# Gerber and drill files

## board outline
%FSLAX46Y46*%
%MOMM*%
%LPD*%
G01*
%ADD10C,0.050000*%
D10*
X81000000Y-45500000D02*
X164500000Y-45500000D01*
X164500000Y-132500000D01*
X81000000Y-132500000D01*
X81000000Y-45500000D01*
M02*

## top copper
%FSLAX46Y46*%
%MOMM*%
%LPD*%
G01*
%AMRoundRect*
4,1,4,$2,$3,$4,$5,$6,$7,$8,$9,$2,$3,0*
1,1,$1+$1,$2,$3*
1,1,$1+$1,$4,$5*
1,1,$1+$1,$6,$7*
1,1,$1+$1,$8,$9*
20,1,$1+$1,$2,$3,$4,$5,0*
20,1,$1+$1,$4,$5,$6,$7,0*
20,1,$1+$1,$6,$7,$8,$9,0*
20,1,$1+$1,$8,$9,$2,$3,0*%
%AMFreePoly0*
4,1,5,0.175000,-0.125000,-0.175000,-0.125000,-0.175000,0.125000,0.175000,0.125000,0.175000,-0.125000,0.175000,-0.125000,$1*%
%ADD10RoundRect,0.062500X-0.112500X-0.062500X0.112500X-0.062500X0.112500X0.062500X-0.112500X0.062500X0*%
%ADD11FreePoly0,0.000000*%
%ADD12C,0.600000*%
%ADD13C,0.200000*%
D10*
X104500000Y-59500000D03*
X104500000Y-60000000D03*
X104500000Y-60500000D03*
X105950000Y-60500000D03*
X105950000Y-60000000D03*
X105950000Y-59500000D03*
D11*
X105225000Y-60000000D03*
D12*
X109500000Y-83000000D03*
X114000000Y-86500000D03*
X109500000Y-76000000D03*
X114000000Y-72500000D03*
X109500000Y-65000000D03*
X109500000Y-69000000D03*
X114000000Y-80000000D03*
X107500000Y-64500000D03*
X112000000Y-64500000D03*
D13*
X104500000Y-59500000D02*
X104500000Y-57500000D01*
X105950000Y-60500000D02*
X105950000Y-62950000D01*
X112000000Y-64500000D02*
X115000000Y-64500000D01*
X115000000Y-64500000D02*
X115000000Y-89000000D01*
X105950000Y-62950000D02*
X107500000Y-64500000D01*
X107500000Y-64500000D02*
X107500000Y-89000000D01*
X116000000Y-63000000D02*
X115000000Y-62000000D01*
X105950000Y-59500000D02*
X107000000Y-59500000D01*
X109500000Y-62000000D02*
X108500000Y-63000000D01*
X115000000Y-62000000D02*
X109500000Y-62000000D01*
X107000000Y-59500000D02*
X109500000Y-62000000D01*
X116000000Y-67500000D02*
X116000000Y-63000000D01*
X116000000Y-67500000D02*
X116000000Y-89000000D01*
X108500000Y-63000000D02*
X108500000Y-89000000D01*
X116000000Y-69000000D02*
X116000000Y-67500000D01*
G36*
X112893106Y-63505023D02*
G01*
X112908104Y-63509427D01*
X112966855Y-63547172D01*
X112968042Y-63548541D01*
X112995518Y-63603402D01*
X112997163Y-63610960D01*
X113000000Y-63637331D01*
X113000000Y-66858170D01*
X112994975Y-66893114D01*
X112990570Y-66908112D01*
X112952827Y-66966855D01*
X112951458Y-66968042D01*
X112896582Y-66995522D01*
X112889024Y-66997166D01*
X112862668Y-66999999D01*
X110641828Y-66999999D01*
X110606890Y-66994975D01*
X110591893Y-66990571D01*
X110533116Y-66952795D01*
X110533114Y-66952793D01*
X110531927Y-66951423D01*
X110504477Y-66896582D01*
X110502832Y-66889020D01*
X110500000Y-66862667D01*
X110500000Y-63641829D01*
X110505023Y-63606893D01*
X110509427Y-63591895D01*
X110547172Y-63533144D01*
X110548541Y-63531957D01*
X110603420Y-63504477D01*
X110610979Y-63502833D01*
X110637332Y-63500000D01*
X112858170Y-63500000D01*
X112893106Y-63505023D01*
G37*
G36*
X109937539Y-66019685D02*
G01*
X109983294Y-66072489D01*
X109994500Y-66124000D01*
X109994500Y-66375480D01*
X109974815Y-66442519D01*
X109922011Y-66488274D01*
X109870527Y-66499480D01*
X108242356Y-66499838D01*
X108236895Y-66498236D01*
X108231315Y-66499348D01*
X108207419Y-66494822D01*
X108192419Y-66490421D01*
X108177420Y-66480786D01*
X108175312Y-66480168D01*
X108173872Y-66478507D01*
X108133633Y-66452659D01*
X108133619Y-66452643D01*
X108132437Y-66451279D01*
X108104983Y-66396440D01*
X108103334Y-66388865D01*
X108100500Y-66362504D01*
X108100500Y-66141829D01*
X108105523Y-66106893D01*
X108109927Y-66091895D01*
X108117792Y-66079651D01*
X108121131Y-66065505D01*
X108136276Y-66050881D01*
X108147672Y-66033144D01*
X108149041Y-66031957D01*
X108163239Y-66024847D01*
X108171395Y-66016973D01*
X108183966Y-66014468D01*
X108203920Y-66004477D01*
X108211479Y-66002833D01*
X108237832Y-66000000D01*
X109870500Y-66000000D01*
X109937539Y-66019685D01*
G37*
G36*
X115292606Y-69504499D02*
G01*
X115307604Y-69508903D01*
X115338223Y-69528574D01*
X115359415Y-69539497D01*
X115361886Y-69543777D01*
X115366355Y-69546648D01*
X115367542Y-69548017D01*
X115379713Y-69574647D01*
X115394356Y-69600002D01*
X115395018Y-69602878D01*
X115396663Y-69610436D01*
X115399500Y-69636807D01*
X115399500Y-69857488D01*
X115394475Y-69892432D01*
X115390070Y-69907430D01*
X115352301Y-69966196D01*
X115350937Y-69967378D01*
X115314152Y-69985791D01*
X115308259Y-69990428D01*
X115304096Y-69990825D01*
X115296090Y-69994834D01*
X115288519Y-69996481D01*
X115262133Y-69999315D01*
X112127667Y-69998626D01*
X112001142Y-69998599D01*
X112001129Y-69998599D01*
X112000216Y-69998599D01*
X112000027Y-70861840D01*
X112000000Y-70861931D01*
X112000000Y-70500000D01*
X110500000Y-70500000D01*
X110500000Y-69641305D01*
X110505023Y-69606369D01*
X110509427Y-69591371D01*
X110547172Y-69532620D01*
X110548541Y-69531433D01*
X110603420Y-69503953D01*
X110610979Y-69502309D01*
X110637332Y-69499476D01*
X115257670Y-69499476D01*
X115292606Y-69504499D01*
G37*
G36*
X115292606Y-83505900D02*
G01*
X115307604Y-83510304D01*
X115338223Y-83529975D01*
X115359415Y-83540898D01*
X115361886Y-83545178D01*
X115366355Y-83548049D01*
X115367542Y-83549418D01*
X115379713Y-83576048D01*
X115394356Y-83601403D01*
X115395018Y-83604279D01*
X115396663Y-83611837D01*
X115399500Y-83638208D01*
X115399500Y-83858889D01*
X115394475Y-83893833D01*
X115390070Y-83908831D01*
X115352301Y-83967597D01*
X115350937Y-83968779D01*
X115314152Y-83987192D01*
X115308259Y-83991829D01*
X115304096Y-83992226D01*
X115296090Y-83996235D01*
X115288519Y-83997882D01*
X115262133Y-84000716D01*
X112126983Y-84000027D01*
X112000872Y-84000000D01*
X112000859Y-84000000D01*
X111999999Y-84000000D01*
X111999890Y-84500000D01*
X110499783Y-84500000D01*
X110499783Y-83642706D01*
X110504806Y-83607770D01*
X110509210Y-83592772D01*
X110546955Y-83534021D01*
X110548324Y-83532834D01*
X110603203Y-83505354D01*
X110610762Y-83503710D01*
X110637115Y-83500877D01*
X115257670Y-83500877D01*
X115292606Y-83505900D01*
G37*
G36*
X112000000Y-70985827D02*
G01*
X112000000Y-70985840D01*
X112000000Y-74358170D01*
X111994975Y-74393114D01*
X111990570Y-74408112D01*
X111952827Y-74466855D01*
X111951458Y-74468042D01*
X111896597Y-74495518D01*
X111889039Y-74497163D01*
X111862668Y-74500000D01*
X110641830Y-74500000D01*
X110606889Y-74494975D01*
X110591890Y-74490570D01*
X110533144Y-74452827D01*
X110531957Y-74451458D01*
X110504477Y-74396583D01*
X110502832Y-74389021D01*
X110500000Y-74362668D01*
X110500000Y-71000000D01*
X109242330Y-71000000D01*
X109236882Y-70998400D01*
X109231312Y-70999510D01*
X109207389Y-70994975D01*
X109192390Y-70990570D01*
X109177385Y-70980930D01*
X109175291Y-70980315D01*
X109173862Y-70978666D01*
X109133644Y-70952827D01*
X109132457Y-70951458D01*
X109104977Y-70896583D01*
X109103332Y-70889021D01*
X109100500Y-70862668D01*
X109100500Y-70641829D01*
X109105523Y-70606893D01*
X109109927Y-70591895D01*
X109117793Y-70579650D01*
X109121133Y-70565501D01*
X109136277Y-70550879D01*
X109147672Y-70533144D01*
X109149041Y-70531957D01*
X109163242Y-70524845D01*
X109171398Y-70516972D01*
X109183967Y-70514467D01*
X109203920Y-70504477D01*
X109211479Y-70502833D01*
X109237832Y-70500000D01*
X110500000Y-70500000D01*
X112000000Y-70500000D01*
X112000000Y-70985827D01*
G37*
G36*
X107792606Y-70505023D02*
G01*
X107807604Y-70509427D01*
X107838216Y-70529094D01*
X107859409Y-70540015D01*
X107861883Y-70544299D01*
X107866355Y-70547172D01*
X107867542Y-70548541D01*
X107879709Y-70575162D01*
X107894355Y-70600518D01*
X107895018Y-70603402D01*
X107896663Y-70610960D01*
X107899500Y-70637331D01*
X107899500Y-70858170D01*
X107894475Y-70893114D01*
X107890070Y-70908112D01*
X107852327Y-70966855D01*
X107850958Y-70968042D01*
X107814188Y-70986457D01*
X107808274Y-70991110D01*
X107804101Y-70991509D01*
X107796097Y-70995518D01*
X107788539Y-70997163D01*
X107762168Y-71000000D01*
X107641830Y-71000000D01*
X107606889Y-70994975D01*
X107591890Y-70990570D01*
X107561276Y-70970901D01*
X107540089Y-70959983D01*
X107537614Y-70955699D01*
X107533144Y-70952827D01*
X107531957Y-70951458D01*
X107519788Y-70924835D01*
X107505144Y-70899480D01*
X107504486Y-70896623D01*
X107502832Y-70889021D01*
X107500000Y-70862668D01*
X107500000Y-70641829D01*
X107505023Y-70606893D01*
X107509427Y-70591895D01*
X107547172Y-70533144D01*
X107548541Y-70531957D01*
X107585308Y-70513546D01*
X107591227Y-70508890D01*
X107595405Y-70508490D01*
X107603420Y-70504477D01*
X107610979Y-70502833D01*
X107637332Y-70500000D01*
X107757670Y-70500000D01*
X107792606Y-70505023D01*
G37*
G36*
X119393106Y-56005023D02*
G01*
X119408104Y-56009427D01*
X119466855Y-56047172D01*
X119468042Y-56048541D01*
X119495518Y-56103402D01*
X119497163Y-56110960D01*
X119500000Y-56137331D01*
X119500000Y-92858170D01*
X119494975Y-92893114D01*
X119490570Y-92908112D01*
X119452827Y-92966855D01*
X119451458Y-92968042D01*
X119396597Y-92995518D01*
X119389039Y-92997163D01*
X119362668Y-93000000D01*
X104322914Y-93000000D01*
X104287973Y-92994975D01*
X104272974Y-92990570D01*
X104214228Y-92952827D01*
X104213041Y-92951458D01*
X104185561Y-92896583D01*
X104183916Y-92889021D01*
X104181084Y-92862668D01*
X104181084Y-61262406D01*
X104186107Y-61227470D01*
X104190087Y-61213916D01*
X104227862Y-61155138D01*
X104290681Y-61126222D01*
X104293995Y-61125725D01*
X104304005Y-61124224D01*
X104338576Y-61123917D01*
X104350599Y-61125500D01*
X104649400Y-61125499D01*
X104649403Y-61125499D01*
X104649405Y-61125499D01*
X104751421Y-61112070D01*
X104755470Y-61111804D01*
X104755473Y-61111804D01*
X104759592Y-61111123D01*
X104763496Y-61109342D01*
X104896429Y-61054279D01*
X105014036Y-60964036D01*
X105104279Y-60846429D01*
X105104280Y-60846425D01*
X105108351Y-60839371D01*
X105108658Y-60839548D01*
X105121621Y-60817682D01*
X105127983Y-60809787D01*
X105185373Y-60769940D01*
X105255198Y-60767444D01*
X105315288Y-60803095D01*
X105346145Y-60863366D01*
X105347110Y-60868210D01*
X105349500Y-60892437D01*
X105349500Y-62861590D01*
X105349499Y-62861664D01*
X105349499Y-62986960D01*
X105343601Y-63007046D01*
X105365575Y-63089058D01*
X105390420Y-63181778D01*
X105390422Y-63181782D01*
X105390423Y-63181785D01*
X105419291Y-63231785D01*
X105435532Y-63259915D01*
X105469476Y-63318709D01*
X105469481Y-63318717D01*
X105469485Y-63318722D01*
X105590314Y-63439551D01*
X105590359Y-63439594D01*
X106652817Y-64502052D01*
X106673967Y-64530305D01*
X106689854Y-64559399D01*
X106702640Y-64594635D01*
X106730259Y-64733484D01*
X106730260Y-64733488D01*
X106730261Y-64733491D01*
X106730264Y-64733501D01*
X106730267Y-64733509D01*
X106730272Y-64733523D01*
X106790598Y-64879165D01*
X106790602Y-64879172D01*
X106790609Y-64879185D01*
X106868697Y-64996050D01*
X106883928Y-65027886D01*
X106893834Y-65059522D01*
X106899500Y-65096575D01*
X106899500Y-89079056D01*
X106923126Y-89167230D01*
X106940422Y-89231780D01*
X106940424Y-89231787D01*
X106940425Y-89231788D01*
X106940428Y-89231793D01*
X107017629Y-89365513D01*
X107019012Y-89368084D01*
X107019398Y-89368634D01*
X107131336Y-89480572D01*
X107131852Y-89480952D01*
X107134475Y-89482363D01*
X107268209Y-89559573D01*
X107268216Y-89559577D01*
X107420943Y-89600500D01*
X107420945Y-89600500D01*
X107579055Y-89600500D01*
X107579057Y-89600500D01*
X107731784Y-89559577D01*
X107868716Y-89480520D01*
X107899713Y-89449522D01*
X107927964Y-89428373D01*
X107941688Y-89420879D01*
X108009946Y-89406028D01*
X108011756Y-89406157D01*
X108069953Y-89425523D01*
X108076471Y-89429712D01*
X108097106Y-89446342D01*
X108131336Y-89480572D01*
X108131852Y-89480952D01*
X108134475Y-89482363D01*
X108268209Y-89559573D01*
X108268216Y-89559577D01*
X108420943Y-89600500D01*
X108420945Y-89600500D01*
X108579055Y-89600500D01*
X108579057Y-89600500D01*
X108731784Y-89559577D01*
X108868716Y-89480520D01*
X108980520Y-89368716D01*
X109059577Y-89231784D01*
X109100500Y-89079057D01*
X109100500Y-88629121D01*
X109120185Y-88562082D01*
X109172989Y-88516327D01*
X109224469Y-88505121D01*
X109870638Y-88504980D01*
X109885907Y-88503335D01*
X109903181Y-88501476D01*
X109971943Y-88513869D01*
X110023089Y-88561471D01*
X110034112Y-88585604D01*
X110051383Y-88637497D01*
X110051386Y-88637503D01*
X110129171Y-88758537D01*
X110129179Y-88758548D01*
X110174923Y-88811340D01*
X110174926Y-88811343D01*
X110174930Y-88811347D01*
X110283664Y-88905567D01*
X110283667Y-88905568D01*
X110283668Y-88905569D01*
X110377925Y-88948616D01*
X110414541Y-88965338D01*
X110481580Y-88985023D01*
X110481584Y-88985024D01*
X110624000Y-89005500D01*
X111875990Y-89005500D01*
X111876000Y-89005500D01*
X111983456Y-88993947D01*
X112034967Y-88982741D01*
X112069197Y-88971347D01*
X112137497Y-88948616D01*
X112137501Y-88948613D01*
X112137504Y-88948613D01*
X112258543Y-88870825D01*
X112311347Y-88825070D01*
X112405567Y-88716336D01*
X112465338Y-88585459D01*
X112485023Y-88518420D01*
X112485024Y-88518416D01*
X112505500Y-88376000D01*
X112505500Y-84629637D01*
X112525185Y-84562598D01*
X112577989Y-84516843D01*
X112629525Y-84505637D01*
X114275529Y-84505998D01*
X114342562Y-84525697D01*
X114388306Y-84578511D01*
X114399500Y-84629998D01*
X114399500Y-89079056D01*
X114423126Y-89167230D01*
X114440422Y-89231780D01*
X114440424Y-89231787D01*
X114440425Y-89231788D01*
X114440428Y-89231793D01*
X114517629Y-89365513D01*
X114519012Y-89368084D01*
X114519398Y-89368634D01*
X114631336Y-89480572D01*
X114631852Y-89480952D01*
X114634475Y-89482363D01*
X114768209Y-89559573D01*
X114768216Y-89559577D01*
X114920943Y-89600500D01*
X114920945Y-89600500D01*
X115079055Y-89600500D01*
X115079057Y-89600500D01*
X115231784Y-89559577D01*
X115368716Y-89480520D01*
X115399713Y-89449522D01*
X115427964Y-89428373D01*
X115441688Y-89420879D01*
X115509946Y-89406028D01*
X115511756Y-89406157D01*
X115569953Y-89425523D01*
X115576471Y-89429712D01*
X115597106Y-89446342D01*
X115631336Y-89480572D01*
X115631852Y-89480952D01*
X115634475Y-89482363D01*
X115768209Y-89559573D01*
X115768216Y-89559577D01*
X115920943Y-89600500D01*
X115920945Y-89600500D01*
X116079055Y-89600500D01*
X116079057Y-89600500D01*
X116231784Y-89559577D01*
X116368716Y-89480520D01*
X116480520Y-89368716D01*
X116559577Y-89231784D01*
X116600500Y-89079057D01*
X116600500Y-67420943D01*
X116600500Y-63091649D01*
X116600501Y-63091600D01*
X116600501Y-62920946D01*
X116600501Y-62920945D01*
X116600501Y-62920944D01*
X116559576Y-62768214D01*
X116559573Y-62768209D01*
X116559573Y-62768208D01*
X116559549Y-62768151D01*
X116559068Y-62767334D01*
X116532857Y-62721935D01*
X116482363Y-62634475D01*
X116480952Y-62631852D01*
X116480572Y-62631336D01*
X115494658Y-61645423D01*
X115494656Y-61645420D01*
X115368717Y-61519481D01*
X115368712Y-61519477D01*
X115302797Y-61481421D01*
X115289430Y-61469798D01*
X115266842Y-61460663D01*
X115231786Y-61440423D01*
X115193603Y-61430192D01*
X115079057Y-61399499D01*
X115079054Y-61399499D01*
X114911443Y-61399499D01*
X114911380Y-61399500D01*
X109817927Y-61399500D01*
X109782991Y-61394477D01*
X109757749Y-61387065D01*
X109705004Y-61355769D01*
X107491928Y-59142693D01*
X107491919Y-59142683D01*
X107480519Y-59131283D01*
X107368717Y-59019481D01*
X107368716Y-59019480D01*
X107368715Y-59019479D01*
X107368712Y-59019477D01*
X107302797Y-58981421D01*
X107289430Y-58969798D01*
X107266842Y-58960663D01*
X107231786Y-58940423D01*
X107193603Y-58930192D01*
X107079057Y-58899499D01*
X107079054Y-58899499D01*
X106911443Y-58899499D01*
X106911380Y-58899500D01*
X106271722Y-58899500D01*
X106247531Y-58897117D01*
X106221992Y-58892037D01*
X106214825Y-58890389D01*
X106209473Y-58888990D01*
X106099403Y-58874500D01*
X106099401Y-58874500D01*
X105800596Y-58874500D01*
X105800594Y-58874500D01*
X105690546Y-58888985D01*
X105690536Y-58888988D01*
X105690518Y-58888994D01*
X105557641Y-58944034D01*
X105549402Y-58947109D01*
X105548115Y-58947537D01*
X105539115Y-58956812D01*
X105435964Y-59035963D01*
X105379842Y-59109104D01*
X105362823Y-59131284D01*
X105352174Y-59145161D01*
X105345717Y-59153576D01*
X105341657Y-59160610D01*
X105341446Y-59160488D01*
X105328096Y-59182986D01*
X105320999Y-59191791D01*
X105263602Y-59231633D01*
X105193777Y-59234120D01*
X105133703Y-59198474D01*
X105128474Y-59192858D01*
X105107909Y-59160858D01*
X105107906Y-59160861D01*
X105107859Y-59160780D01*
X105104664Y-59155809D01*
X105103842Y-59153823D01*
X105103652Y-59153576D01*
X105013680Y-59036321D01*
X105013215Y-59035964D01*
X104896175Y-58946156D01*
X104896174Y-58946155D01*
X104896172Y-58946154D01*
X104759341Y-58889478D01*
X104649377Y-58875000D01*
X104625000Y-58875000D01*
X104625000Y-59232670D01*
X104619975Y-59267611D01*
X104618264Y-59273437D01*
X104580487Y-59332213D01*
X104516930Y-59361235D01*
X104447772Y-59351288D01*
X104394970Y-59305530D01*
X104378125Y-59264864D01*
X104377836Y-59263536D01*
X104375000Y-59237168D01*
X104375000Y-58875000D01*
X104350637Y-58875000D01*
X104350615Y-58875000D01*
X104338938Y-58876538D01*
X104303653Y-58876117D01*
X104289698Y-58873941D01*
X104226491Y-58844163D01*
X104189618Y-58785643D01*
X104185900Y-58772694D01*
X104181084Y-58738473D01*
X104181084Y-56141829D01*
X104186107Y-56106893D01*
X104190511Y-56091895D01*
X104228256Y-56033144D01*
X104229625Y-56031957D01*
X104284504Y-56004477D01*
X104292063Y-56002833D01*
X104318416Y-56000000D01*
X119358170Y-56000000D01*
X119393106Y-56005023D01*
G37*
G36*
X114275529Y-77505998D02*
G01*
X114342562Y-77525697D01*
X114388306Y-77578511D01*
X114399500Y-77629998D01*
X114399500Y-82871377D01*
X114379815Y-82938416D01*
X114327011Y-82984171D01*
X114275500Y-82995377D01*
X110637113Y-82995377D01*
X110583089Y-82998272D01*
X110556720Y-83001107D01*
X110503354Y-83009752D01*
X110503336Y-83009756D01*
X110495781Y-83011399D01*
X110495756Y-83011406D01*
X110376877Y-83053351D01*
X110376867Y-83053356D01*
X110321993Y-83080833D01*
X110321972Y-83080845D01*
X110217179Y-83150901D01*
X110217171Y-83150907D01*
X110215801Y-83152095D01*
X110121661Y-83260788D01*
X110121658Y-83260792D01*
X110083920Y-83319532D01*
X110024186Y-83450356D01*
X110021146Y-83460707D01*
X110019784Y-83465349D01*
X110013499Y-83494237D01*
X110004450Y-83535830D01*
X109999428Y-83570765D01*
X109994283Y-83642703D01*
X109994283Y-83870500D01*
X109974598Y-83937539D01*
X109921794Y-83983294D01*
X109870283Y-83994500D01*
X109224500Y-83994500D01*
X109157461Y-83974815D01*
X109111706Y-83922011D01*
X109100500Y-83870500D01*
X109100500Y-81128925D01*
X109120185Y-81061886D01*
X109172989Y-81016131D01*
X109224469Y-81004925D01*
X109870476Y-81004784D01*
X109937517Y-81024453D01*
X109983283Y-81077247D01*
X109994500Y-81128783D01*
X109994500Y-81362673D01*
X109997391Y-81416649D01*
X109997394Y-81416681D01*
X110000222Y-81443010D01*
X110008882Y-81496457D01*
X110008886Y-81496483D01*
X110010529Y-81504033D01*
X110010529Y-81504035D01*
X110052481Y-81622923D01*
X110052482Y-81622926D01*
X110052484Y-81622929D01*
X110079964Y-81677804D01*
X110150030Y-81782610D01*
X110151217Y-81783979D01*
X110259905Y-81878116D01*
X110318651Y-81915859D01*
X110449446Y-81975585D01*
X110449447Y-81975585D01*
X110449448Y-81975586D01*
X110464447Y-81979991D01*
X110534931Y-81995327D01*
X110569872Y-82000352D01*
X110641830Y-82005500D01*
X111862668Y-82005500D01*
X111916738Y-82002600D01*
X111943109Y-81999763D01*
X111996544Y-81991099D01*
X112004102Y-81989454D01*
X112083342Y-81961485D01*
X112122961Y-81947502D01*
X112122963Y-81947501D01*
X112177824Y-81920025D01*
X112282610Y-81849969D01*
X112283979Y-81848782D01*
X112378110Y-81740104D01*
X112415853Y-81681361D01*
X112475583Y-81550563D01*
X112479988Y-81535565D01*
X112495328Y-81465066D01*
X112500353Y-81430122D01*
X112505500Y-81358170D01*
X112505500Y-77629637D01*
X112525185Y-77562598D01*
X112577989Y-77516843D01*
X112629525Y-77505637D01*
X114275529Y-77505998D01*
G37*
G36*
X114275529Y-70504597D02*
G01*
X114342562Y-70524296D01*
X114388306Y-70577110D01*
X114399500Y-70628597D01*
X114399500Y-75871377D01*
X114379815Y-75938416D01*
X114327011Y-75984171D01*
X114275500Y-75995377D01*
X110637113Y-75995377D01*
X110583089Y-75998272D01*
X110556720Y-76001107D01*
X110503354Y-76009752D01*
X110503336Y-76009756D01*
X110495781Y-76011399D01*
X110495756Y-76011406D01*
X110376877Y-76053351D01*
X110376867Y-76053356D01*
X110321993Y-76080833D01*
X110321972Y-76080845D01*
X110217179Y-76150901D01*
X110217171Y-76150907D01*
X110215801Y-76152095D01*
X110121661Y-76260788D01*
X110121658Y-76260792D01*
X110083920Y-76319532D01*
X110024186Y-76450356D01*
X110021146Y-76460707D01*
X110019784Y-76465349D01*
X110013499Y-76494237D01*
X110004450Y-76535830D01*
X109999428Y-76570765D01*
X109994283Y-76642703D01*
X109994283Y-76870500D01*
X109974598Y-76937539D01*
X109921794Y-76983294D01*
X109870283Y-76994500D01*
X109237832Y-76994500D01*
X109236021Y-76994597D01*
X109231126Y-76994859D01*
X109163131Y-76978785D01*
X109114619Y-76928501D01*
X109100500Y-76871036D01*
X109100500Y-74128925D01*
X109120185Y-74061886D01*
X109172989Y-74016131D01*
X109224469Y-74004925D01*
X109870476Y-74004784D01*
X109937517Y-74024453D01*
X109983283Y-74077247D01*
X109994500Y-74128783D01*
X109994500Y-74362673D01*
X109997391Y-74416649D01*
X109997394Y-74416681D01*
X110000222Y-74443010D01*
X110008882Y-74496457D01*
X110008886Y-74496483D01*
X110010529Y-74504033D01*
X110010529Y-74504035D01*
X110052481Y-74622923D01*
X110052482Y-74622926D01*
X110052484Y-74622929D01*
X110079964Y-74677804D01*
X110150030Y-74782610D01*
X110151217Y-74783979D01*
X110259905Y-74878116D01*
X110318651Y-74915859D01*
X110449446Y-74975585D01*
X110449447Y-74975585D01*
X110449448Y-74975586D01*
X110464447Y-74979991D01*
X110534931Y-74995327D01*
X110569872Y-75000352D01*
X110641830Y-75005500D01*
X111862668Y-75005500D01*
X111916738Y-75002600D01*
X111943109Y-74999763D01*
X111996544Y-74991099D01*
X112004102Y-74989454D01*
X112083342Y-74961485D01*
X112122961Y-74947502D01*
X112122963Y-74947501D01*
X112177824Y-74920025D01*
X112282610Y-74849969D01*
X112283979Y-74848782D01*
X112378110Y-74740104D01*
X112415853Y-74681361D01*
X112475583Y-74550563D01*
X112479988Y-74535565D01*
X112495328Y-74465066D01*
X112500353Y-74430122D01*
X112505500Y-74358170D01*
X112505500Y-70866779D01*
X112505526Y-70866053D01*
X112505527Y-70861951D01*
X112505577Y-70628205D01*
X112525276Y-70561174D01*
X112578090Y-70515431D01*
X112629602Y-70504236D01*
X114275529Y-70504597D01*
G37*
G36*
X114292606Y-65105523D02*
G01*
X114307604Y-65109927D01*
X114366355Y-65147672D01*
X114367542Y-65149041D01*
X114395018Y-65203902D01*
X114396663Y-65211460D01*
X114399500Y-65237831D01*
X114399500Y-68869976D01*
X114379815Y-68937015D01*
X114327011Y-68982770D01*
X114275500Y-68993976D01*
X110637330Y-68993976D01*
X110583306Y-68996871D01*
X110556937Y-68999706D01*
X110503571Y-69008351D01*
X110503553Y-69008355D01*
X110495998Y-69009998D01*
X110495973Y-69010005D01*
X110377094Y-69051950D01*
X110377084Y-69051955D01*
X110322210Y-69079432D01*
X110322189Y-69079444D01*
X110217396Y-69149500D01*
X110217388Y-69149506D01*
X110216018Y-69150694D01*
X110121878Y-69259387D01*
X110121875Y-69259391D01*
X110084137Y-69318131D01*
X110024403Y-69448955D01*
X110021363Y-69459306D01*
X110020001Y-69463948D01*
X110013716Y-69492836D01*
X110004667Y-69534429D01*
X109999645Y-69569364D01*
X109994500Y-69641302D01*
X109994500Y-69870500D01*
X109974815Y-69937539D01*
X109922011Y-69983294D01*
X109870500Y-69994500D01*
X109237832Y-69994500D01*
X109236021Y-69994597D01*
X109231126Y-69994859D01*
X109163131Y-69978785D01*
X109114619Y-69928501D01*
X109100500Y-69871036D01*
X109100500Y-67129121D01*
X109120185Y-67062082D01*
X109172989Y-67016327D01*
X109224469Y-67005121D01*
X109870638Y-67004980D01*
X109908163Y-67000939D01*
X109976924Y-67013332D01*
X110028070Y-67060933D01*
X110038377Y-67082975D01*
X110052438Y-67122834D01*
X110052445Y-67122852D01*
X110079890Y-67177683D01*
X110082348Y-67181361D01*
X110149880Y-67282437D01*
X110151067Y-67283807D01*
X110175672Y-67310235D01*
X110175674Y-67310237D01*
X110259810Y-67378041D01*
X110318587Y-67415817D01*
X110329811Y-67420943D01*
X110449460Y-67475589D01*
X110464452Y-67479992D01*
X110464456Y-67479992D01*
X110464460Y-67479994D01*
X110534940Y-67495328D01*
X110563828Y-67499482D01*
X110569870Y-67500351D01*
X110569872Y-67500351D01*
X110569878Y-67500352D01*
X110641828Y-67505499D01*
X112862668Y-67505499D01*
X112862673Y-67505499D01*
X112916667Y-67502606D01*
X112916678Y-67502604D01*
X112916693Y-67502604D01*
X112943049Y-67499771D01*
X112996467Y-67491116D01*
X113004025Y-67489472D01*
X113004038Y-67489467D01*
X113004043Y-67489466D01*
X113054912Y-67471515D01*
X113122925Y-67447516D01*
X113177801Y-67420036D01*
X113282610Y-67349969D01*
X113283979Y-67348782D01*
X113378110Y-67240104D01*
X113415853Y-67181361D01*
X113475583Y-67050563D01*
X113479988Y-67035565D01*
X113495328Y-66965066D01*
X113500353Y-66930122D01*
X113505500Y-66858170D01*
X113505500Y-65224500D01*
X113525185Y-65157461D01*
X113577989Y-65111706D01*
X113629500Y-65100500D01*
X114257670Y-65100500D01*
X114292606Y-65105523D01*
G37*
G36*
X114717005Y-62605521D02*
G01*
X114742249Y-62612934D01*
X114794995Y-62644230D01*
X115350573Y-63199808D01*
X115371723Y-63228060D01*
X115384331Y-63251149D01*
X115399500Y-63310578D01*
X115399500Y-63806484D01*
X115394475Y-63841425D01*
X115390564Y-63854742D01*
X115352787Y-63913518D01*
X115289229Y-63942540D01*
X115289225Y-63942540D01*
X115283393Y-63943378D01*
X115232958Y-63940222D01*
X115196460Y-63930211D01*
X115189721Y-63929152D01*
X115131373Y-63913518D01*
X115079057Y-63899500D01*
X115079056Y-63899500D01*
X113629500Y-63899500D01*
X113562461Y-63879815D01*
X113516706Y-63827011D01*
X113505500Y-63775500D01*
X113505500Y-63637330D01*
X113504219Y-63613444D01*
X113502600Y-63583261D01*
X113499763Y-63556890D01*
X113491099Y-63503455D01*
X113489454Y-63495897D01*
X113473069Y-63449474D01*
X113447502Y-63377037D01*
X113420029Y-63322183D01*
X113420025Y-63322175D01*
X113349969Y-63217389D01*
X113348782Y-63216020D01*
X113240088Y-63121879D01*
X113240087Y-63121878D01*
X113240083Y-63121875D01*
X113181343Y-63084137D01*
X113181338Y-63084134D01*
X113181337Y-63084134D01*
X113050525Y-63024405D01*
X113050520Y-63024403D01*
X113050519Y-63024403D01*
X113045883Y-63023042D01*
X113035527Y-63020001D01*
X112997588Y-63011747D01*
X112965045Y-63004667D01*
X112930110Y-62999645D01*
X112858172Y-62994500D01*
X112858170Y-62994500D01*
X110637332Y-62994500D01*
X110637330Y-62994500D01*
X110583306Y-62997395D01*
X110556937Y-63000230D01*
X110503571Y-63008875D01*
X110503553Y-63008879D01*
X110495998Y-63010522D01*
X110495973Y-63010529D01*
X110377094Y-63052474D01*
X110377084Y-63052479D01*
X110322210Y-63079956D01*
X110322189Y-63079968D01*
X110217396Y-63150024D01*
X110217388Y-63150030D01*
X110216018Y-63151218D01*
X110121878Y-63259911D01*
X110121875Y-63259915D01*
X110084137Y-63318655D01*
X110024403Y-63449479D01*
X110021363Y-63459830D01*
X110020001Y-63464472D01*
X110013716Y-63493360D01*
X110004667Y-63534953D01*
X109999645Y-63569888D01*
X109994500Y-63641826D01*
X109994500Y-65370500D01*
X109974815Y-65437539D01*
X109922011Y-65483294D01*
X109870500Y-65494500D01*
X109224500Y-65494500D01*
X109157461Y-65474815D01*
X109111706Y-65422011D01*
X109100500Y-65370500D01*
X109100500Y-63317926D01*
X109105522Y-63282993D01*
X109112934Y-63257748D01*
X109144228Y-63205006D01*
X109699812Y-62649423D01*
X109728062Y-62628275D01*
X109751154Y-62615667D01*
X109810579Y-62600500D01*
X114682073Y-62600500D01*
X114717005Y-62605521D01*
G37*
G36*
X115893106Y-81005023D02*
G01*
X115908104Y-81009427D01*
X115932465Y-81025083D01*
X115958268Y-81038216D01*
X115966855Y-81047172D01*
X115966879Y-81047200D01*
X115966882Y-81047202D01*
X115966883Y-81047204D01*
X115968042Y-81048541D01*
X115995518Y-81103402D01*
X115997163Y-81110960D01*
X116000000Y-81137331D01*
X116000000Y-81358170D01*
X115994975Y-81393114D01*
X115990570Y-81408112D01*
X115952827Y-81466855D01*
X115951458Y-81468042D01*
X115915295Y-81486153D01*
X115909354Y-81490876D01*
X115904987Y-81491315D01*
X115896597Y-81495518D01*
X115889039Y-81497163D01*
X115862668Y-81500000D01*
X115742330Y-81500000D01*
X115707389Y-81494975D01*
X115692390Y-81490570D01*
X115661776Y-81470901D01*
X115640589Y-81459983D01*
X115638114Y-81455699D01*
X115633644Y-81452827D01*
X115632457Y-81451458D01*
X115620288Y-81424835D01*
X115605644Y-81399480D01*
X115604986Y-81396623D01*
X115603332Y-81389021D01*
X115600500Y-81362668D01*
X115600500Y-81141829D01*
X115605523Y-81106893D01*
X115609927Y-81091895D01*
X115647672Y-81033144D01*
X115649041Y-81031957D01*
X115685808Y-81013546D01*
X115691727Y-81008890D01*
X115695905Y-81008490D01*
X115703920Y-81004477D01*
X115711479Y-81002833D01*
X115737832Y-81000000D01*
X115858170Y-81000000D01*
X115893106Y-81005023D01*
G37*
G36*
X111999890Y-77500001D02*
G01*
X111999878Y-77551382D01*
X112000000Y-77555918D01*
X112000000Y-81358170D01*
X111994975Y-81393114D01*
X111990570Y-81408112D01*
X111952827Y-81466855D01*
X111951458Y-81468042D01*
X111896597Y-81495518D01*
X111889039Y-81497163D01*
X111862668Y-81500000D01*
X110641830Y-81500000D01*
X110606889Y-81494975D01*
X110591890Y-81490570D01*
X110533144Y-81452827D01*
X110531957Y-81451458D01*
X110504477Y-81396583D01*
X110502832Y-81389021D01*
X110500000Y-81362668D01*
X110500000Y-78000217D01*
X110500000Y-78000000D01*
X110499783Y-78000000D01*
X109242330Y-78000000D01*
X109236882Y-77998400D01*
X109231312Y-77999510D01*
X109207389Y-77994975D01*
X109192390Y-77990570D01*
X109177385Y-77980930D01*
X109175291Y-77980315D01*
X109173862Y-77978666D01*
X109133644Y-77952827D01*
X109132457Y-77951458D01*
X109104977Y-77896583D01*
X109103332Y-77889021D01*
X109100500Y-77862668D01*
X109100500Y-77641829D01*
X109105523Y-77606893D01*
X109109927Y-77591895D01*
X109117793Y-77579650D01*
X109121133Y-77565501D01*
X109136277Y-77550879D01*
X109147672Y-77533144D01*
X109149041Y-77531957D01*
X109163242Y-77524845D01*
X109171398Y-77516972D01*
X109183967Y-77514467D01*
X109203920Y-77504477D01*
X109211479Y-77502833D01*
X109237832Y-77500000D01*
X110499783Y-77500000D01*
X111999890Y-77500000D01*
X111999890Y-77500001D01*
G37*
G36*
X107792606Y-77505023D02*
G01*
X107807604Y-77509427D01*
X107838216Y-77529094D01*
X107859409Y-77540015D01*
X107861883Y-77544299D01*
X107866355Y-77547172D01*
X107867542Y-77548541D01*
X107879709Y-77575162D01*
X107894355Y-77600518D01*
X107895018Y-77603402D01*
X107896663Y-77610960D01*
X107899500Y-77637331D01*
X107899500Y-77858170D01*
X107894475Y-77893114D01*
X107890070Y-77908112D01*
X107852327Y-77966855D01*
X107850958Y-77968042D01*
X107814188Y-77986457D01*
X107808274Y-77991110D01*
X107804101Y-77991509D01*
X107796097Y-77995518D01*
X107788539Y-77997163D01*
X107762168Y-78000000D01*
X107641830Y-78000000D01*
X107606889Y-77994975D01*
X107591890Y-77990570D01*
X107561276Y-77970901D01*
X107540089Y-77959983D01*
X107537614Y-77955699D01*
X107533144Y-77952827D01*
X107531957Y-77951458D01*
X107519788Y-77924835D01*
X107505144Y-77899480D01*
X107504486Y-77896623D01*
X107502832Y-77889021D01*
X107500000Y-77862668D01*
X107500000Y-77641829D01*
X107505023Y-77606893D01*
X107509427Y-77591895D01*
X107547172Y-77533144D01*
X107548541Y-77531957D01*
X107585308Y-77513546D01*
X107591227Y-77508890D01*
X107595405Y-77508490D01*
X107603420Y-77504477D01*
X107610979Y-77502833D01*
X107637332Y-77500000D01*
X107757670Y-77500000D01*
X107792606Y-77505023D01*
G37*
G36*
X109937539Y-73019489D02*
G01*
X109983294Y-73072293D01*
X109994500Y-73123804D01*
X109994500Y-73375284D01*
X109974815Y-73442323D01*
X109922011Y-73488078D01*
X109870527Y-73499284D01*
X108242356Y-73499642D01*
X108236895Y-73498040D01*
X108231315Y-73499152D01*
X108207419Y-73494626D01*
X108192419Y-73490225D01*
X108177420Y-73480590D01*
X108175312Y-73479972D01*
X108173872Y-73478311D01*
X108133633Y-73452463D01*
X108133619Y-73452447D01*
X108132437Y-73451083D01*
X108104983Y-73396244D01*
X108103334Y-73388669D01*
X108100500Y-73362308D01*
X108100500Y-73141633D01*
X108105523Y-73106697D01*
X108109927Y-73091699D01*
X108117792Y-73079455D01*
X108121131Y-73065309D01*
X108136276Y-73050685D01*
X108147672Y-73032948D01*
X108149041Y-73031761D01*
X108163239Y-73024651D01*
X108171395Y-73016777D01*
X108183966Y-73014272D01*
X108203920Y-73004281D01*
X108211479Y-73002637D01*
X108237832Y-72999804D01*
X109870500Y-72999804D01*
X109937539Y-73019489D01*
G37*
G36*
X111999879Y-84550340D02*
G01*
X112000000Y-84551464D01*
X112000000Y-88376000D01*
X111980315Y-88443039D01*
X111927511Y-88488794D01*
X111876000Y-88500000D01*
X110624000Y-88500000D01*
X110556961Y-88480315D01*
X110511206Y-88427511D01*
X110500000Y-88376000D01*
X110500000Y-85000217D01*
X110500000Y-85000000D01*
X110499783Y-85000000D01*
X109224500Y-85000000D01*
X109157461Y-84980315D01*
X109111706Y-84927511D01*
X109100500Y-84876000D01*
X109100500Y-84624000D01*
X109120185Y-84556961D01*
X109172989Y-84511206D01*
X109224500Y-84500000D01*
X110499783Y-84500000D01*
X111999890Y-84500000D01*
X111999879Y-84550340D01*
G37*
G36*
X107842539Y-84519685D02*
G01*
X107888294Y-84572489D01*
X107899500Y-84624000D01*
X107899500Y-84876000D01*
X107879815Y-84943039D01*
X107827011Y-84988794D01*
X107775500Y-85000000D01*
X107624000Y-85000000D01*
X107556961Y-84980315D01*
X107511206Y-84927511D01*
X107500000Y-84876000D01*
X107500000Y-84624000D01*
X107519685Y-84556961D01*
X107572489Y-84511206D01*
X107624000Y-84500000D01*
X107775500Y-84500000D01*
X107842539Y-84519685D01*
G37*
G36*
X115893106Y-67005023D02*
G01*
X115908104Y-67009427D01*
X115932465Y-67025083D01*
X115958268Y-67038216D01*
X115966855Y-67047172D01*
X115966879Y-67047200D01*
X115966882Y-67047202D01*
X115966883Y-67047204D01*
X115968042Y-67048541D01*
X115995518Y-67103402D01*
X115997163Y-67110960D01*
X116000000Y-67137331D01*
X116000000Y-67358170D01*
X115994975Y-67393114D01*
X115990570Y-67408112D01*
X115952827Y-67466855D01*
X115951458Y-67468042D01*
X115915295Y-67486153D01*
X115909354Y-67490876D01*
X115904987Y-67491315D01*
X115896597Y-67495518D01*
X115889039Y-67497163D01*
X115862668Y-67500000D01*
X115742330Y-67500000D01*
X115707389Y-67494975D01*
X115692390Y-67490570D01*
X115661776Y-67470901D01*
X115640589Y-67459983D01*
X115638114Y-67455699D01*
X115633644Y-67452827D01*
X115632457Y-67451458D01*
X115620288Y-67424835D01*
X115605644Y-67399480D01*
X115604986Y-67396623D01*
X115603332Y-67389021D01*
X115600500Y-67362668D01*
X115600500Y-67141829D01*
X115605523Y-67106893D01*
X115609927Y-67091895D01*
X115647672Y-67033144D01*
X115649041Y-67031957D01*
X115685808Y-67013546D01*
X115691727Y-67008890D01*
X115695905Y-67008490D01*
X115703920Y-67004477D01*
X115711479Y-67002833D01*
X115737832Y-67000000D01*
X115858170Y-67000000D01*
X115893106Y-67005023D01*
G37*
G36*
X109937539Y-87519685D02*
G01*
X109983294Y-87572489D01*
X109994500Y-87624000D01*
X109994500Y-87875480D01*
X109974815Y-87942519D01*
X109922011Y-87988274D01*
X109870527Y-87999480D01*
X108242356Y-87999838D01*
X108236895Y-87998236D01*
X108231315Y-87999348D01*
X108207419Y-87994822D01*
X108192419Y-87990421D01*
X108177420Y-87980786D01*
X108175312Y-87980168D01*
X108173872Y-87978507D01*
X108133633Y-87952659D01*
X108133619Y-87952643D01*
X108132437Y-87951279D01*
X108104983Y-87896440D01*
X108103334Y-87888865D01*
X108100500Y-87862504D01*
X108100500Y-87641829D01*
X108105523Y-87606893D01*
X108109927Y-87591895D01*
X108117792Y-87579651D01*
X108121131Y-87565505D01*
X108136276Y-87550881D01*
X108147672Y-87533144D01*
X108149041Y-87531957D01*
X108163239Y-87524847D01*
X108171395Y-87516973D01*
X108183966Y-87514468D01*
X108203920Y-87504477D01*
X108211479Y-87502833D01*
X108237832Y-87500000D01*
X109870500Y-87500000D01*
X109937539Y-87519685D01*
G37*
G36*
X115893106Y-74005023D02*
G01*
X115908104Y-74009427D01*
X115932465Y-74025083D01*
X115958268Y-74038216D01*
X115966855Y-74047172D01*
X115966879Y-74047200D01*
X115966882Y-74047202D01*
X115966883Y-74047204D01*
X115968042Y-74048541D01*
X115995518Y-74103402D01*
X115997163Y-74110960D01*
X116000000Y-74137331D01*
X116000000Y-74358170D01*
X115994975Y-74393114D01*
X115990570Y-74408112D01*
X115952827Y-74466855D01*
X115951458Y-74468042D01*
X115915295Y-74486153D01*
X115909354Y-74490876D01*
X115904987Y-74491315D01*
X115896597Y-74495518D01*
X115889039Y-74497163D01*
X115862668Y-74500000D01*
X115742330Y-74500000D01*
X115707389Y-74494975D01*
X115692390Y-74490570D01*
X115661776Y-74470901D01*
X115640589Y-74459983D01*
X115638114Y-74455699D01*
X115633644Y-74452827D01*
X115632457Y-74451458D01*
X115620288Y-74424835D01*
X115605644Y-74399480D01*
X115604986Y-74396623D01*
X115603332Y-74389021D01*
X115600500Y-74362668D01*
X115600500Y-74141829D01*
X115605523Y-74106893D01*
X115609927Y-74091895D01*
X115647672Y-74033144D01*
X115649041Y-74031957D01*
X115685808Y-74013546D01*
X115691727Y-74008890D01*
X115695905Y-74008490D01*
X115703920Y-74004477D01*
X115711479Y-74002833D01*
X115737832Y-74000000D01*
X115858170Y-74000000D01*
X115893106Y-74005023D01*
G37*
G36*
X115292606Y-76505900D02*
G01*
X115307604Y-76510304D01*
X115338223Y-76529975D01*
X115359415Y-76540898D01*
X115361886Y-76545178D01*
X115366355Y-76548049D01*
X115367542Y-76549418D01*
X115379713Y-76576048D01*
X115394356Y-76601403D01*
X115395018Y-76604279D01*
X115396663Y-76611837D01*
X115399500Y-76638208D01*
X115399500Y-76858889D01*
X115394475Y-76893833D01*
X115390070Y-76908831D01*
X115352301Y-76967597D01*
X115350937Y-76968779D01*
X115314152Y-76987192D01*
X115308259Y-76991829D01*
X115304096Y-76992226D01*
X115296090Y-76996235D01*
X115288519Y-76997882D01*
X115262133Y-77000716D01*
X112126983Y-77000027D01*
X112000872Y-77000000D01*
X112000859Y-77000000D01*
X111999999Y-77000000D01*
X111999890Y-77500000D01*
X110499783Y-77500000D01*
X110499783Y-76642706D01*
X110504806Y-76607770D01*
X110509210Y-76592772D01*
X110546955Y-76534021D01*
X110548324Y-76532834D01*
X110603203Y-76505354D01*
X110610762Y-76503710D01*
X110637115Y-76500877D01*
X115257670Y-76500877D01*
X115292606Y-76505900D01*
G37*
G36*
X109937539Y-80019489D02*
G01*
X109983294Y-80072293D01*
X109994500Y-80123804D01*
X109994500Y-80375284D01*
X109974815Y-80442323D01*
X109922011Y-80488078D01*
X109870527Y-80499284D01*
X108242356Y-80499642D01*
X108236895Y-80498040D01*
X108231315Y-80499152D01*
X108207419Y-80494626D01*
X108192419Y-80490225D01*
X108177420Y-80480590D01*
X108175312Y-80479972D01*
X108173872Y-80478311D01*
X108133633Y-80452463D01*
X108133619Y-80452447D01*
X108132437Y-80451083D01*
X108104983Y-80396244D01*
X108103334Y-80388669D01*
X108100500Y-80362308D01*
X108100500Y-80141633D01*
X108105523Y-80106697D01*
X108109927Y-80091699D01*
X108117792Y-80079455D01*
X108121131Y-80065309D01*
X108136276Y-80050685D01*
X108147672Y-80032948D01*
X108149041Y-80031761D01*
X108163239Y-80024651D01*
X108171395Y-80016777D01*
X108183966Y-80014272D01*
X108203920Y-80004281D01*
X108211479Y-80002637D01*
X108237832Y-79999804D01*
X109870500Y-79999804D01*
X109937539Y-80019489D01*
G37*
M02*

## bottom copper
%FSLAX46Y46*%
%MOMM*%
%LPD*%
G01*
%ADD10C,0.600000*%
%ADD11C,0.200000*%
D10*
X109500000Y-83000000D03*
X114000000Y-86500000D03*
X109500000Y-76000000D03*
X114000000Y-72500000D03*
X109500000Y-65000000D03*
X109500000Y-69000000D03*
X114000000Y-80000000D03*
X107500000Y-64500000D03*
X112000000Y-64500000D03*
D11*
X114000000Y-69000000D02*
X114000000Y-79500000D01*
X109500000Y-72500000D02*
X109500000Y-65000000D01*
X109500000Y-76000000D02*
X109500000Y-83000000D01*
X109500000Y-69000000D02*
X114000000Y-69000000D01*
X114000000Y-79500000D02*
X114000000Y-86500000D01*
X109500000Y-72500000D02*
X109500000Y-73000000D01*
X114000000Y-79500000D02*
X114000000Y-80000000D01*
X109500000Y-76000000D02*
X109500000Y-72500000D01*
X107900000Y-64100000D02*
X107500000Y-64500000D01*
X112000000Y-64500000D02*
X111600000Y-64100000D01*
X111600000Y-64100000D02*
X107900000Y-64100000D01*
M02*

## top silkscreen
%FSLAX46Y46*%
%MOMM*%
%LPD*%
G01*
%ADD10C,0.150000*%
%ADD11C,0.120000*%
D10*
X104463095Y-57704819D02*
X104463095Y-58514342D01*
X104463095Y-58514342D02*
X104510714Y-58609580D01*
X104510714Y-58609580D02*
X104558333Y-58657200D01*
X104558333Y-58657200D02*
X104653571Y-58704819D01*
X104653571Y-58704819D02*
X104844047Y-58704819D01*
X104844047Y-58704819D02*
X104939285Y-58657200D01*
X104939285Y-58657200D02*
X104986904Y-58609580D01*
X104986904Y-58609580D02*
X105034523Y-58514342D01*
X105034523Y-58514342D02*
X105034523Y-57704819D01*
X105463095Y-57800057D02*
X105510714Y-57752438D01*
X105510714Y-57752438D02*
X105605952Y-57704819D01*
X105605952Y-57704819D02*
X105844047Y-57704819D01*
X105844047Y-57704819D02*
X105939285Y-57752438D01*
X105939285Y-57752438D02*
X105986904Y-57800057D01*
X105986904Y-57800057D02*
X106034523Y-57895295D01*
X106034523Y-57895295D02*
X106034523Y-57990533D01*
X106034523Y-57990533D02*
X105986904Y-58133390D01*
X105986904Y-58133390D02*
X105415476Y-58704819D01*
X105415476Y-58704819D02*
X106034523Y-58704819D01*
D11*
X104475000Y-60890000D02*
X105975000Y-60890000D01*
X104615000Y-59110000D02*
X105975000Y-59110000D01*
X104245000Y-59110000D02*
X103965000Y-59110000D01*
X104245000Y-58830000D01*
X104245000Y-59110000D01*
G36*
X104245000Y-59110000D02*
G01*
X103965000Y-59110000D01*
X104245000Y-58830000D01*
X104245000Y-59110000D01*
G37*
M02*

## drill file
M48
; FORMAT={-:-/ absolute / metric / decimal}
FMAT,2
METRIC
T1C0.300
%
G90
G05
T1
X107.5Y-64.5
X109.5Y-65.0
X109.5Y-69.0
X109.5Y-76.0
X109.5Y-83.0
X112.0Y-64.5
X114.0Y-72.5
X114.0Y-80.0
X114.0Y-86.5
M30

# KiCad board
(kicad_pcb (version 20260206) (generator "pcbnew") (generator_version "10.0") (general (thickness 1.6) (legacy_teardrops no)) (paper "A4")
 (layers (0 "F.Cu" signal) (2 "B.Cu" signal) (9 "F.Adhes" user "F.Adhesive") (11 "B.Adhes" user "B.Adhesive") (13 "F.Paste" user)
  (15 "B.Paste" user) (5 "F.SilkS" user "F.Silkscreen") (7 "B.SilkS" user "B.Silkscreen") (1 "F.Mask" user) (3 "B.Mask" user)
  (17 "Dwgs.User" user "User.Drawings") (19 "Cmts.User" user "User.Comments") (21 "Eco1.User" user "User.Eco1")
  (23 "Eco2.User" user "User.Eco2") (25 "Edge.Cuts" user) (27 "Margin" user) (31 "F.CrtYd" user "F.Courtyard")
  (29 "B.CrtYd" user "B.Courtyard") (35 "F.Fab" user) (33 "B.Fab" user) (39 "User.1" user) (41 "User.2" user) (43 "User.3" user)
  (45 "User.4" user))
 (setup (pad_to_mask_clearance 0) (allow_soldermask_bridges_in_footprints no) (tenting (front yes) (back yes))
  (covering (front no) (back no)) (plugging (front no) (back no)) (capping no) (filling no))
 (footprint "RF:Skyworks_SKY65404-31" (layer "F.Cu") (at 105.225 60)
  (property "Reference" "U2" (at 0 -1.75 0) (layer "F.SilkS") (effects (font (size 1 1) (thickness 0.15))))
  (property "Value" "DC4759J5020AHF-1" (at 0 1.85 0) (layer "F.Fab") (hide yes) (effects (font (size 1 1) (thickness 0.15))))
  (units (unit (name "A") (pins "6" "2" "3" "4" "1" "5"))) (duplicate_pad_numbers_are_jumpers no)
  (fp_line (start -0.75 0.89) (end 0.75 0.89) (stroke (width 0.12) (type solid)) (layer "F.SilkS"))
  (fp_line (start -0.61 -0.89) (end 0.75 -0.89) (stroke (width 0.12) (type solid)) (layer "F.SilkS"))
  (fp_poly
   (pts (xy -0.98 -0.89) (xy -1.26 -0.89) (xy -0.98 -1.17) (xy -0.98 -0.89)) (stroke (width 0.12) (type solid)) (fill yes) (layer "F.SilkS"))
  (pad "1" smd roundrect (at -0.725 -0.5) (size 0.35 0.25) (layers "F.Cu" "F.Mask" "F.Paste") (roundrect_rratio 0.25)
   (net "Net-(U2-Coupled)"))
  (pad "2" smd roundrect (at -0.725 0) (size 0.35 0.25) (layers "F.Cu" "F.Mask" "F.Paste") (roundrect_rratio 0.25) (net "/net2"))
  (pad "3" smd roundrect (at -0.725 0.5) (size 0.35 0.25) (layers "F.Cu" "F.Mask" "F.Paste") (roundrect_rratio 0.25) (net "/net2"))
  (pad "4" smd roundrect (at 0.725 0.5) (size 0.35 0.25) (layers "F.Cu" "F.Mask" "F.Paste") (roundrect_rratio 0.25) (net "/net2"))
  (pad "5" smd roundrect (at 0.725 0) (size 0.35 0.25) (layers "F.Cu" "F.Mask" "F.Paste") (roundrect_rratio 0.25) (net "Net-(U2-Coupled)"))
  (pad "6" smd roundrect (at 0.725 -0.5) (size 0.35 0.25) (layers "F.Cu" "F.Mask" "F.Paste") (roundrect_rratio 0.25) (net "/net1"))
  (pad "7" smd custom (at 0 0) (size 0.35 0.25) (layers "F.Cu" "F.Mask" "F.Paste") (zone_connect 0)
   (options (clearance outline) (anchor rect)) (primitives)))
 (gr_rect (start 81 45.5) (end 164.5 132.5) (stroke (width 0.05) (type default)) (fill no) (layer "Edge.Cuts"))
 (segment (start 104.5 59.5) (end 104.5 57.5) (width 0.2) (layer "F.Cu") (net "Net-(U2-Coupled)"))
 (via (at 109.5 83) (size 0.6) (drill 0.3) (layers "F.Cu" "B.Cu") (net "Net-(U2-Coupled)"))
 (via (at 114 86.5) (size 0.6) (drill 0.3) (layers "F.Cu" "B.Cu") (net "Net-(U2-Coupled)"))
 (via (at 109.5 76) (size 0.6) (drill 0.3) (layers "F.Cu" "B.Cu") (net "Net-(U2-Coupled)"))
 (via (at 114 72.5) (size 0.6) (drill 0.3) (layers "F.Cu" "B.Cu") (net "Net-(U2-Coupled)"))
 (via (at 109.5 65) (size 0.6) (drill 0.3) (layers "F.Cu" "B.Cu") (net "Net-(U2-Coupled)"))
 (via (at 109.5 69) (size 0.6) (drill 0.3) (layers "F.Cu" "B.Cu") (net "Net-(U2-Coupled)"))
 (via (at 114 80) (size 0.6) (drill 0.3) (layers "F.Cu" "B.Cu") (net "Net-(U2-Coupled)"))
 (segment (start 114 69) (end 114 79.5) (width 0.2) (layer "B.Cu") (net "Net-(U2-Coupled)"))
 (segment (start 109.5 72.5) (end 109.5 65) (width 0.2) (layer "B.Cu") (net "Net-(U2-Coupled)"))
 (segment (start 109.5 76) (end 109.5 83) (width 0.2) (layer "B.Cu") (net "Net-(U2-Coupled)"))
 (segment (start 109.5 69) (end 114 69) (width 0.2) (layer "B.Cu") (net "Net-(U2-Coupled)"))
 (segment (start 114 79.5) (end 114 86.5) (width 0.2) (layer "B.Cu") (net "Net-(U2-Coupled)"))
 (segment (start 109.5 72.5) (end 109.5 73) (width 0.2) (layer "B.Cu") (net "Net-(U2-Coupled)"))
 (segment (start 114 79.5) (end 114 80) (width 0.2) (layer "B.Cu") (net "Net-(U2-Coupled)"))
 (segment (start 109.5 76) (end 109.5 72.5) (width 0.2) (layer "B.Cu") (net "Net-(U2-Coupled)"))
 (segment (start 105.95 60.5) (end 105.95 62.95) (width 0.2) (layer "F.Cu") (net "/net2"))
 (segment (start 112 64.5) (end 115 64.5) (width 0.2) (layer "F.Cu") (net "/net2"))
 (segment (start 115 64.5) (end 115 89) (width 0.2) (layer "F.Cu") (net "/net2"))
 (segment (start 105.95 62.95) (end 107.5 64.5) (width 0.2) (layer "F.Cu") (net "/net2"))
 (segment (start 107.5 64.5) (end 107.5 89) (width 0.2) (layer "F.Cu") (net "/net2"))
 (via (at 107.5 64.5) (size 0.6) (drill 0.3) (layers "F.Cu" "B.Cu") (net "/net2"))
 (via (at 112 64.5) (size 0.6) (drill 0.3) (layers "F.Cu" "B.Cu") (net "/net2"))
 (segment (start 107.9 64.1) (end 107.5 64.5) (width 0.2) (layer "B.Cu") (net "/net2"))
 (segment (start 112 64.5) (end 111.6 64.1) (width 0.2) (layer "B.Cu") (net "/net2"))
 (segment (start 111.6 64.1) (end 107.9 64.1) (width 0.2) (layer "B.Cu") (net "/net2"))
 (segment (start 116 63) (end 115 62) (width 0.2) (layer "F.Cu") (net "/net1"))
 (segment (start 105.95 59.5) (end 107 59.5) (width 0.2) (layer "F.Cu") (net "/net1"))
 (segment (start 109.5 62) (end 108.5 63) (width 0.2) (layer "F.Cu") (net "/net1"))
 (segment (start 115 62) (end 109.5 62) (width 0.2) (layer "F.Cu") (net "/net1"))
 (segment (start 107 59.5) (end 109.5 62) (width 0.2) (layer "F.Cu") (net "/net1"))
 (segment (start 116 67.5) (end 116 63) (width 0.2) (layer "F.Cu") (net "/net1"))
 (segment (start 116 67.5) (end 116 89) (width 0.2) (layer "F.Cu") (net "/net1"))
 (segment (start 108.5 63) (end 108.5 89) (width 0.2) (layer "F.Cu") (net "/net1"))
 (segment (start 116 69) (end 116 67.5) (width 0.2) (layer "F.Cu") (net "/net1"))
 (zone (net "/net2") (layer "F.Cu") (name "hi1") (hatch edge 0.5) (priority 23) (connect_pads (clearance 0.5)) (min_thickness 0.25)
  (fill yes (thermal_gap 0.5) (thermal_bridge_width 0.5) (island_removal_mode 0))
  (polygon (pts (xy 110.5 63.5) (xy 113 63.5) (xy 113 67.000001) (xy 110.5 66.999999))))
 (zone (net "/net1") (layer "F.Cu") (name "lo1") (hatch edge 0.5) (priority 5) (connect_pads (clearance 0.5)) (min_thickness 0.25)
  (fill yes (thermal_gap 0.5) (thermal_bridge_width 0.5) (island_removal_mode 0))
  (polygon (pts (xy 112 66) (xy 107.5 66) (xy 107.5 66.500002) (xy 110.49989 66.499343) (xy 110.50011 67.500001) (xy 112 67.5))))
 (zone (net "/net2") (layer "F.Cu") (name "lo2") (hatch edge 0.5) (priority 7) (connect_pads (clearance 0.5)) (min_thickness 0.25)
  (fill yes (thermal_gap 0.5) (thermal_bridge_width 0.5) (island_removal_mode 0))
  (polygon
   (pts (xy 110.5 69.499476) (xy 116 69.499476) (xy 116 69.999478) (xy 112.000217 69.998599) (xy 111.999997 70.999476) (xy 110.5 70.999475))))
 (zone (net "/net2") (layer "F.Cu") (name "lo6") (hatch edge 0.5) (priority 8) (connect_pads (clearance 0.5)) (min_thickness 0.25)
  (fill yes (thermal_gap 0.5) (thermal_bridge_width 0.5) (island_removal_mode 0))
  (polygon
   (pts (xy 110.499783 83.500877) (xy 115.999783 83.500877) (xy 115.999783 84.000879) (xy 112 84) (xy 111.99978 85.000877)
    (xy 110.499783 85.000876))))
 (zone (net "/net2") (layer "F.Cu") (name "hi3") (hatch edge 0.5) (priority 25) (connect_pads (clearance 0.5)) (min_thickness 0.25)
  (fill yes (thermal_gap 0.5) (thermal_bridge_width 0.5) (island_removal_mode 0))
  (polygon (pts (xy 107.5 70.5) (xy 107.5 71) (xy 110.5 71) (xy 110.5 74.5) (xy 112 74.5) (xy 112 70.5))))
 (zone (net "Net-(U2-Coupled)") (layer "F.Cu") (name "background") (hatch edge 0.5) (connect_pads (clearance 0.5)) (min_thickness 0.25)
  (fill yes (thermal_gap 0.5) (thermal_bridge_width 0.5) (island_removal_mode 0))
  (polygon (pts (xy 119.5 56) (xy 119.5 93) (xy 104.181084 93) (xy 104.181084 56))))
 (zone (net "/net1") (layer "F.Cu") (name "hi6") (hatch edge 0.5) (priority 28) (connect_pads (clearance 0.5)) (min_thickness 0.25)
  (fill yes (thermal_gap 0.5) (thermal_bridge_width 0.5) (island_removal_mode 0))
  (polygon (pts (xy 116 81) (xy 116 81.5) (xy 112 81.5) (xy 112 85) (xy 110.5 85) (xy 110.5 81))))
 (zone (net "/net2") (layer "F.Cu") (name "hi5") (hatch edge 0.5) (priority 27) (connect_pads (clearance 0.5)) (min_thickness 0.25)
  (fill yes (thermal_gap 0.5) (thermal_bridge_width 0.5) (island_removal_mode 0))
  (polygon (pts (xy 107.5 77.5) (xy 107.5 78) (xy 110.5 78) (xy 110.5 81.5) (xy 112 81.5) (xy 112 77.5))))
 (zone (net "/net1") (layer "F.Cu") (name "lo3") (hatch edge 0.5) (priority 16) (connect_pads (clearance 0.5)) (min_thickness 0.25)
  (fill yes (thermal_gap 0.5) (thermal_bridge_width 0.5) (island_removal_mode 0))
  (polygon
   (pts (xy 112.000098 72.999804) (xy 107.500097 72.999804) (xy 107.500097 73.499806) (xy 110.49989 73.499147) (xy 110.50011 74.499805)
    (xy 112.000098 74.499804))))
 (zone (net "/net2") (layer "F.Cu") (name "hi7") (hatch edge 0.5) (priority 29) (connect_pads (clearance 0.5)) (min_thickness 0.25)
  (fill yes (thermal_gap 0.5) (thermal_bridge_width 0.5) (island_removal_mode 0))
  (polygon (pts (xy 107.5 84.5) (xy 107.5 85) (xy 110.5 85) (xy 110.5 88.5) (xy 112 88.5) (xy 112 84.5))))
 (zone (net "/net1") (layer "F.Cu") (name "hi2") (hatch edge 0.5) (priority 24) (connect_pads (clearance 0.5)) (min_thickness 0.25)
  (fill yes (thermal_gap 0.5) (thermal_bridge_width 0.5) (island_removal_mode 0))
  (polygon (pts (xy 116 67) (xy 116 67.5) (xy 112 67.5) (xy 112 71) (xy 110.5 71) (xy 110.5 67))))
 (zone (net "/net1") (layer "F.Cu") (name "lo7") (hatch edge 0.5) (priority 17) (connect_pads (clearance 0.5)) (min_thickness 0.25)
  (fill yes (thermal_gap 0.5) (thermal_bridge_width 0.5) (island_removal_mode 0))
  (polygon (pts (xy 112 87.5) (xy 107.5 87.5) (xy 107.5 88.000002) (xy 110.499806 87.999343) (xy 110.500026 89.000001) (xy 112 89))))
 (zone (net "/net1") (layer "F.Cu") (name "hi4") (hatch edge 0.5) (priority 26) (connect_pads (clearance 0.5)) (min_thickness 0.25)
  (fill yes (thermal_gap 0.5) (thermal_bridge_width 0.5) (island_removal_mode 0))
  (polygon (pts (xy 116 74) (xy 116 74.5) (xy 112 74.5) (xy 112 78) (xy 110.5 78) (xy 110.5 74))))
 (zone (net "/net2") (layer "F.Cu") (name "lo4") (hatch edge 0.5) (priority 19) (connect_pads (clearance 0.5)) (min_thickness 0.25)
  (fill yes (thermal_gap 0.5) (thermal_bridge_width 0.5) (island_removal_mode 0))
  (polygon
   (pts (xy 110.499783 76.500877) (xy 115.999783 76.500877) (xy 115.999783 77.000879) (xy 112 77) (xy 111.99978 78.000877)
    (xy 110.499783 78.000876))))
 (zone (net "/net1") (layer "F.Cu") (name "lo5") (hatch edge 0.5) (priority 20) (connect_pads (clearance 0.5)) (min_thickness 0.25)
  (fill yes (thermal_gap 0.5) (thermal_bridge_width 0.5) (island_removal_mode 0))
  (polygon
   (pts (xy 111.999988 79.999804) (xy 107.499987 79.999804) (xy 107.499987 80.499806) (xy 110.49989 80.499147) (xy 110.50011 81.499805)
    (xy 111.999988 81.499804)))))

